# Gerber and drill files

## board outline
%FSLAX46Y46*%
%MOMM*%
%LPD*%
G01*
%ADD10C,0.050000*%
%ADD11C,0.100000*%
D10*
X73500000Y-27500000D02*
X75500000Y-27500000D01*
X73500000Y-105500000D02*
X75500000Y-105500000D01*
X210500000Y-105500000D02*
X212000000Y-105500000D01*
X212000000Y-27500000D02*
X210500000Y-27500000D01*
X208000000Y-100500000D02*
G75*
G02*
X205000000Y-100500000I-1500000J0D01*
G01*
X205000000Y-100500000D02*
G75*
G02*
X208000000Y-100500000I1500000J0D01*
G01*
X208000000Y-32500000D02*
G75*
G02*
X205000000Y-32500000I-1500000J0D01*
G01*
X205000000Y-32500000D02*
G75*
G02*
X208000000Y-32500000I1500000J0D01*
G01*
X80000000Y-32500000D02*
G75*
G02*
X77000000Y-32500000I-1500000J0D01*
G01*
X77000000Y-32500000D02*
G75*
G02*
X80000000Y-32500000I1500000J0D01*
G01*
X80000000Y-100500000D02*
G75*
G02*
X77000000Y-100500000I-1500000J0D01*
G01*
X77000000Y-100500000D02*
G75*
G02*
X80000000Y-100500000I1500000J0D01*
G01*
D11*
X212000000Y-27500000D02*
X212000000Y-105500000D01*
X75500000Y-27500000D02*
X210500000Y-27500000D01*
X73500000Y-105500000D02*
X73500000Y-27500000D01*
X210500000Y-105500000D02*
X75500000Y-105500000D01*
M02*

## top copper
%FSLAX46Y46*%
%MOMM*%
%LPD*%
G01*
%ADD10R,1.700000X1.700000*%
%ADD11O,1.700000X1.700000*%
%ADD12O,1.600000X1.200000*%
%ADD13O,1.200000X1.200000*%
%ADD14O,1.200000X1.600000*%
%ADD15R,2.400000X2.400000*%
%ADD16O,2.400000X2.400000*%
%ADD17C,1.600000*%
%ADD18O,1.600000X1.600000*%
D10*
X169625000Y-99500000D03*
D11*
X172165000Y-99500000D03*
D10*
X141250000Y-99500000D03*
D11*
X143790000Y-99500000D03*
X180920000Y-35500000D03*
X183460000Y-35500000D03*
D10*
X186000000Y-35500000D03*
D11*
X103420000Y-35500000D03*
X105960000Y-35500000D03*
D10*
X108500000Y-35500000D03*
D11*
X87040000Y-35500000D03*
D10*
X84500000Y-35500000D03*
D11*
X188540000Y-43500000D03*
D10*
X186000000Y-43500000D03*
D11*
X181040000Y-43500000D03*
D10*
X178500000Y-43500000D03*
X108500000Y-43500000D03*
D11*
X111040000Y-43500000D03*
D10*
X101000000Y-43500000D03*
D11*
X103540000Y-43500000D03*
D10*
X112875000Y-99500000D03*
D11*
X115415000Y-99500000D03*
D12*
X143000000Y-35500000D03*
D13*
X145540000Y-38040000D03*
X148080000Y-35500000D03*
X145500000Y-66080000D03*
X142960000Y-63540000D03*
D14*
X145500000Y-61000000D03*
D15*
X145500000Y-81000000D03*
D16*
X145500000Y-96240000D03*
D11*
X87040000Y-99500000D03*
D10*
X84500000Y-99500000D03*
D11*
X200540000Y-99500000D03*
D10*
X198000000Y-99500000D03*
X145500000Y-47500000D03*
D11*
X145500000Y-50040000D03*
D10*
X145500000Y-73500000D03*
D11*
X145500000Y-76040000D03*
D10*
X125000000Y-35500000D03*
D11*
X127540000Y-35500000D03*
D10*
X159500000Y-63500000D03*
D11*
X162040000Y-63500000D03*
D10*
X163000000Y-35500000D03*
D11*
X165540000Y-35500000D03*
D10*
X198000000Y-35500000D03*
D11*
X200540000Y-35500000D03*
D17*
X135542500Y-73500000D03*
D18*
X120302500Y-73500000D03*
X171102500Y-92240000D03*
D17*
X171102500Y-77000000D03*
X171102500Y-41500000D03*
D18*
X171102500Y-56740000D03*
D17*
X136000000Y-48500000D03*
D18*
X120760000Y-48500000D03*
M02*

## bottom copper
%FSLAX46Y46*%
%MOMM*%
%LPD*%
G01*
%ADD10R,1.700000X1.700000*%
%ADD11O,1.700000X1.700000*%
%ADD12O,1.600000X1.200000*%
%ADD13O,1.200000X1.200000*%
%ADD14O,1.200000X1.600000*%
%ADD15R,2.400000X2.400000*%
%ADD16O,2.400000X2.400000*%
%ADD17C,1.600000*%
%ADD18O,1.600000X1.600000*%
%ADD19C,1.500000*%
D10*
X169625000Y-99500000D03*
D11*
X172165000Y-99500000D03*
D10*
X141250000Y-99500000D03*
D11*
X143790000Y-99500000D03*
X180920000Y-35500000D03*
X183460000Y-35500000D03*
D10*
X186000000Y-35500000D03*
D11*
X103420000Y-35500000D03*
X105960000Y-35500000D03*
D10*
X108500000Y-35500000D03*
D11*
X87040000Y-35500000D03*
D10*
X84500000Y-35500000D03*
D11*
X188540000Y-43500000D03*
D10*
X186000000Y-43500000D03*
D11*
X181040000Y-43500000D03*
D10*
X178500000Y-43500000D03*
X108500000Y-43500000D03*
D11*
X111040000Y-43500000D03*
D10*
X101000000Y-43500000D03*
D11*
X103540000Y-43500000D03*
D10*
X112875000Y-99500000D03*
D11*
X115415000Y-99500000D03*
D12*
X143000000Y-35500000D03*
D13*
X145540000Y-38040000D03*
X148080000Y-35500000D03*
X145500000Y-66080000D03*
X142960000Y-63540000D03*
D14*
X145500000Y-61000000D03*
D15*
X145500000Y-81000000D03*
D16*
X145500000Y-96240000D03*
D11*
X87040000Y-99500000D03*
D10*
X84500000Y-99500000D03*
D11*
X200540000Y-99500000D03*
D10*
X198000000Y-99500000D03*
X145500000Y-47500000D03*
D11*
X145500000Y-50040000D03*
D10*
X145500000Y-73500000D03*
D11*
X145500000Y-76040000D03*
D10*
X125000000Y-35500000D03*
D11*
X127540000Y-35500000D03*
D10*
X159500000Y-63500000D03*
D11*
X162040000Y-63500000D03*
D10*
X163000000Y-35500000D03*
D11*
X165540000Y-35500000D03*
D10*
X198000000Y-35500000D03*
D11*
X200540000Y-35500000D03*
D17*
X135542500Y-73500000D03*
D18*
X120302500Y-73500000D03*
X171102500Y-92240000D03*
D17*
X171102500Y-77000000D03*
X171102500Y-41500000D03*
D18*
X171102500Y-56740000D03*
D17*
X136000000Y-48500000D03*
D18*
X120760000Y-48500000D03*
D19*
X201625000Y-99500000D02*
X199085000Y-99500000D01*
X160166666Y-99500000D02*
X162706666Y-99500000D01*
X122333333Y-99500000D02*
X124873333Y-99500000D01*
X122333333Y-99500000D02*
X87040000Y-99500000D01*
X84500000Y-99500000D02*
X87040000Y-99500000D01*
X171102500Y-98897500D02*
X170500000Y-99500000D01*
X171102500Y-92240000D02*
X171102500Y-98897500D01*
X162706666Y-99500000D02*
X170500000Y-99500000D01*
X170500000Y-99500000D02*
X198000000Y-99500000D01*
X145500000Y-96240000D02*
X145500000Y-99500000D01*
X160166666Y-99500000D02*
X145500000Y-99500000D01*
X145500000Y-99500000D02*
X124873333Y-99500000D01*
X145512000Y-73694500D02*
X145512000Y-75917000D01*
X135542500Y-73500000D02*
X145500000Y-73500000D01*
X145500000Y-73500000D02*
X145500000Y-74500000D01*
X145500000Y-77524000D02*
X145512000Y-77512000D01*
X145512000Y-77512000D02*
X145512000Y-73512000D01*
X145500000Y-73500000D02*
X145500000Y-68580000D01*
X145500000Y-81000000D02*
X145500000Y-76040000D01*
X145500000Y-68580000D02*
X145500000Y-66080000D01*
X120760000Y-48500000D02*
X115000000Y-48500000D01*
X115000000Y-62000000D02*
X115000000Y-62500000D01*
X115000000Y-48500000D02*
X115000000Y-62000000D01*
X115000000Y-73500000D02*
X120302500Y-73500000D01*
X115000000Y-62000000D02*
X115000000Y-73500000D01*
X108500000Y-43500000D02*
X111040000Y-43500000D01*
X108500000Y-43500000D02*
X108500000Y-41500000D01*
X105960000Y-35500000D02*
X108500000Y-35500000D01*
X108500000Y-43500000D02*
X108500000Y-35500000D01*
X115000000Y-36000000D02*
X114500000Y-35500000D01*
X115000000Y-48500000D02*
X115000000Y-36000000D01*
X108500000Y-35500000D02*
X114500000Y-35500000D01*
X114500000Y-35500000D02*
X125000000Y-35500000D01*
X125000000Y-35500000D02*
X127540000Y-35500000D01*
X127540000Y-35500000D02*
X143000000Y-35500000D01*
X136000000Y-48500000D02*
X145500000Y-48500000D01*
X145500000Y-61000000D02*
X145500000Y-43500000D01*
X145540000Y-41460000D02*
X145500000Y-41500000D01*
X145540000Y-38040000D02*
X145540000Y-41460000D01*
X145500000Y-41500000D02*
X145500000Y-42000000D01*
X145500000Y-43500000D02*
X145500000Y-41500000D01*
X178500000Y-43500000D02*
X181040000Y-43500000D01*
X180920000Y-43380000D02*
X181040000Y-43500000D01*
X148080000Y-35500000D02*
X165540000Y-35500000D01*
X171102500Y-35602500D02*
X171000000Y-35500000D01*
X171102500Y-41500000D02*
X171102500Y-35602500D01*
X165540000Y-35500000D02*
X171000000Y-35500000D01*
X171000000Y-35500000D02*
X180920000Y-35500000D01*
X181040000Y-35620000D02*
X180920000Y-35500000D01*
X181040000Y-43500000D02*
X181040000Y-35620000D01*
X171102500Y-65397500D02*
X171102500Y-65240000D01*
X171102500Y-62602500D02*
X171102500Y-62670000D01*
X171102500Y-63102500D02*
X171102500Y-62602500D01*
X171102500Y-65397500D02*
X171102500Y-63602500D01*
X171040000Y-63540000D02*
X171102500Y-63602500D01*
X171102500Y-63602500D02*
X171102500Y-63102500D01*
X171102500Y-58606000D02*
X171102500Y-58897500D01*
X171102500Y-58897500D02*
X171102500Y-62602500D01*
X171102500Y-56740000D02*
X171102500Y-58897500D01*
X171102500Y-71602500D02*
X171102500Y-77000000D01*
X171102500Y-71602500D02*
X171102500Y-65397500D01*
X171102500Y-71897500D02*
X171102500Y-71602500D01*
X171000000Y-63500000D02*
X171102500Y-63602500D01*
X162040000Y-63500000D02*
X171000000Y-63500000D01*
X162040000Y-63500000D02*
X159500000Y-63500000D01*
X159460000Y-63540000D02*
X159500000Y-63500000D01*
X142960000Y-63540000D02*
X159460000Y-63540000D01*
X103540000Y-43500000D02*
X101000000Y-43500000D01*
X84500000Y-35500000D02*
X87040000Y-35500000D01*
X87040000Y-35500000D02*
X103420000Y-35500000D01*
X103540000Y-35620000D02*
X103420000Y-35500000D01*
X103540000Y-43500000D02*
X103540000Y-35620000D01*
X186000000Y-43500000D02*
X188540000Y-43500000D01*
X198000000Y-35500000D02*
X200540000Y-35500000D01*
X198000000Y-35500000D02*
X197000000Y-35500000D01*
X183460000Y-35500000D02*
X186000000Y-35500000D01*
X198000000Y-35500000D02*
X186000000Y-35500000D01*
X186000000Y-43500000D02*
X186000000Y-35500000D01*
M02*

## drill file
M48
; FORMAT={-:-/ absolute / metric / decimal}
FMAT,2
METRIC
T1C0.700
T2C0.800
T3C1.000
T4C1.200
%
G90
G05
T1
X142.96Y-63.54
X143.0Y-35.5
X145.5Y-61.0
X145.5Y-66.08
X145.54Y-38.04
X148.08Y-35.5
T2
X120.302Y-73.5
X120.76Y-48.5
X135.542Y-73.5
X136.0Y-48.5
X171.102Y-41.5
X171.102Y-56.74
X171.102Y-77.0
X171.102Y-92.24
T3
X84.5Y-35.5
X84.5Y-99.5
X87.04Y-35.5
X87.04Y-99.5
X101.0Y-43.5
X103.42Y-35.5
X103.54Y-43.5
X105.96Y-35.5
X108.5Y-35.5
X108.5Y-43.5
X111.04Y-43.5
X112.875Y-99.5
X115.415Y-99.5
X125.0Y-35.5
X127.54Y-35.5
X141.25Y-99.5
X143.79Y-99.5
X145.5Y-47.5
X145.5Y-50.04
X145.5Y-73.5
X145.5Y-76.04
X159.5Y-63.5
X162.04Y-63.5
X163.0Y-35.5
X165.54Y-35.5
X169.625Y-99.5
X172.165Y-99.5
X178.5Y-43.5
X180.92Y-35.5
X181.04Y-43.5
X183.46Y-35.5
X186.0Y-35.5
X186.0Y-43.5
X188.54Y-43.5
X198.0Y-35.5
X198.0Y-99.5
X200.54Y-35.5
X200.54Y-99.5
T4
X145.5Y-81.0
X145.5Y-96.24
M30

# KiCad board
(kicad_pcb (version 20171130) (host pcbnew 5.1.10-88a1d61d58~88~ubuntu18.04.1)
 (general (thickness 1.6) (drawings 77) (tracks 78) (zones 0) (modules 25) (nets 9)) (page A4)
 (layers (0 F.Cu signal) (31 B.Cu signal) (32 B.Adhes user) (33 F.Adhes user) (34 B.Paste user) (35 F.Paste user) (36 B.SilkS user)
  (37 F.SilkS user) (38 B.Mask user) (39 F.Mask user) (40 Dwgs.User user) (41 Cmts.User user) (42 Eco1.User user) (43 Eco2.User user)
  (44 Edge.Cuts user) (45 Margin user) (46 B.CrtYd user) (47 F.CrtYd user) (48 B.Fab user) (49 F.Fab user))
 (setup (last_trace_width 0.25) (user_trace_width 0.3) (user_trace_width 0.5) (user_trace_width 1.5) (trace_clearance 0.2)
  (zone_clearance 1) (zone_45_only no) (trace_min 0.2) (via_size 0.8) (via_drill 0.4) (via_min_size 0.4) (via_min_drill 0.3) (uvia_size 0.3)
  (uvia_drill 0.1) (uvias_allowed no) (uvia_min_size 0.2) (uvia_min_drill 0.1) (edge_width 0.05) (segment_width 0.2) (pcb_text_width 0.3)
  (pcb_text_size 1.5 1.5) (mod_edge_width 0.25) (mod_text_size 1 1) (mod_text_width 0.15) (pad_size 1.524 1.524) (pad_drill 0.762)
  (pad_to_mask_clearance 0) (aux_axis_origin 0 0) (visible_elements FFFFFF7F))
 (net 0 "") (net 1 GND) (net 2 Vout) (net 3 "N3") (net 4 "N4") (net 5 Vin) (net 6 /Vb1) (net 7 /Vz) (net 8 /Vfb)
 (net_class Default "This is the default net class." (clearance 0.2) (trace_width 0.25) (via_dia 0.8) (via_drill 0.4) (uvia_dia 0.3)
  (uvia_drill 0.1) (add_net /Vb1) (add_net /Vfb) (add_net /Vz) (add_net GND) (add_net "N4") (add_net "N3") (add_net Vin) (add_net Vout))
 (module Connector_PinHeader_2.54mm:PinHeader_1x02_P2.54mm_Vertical (layer F.Cu) (at 169.625 99.5 90)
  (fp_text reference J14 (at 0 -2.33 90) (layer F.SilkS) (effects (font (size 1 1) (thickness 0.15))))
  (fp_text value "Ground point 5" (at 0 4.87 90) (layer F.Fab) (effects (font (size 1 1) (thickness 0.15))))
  (pad 1 thru_hole rect (at 0 0 90) (size 1.7 1.7) (drill 1) (layers *.Cu *.Mask) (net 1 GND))
  (pad 2 thru_hole oval (at 0 2.54 90) (size 1.7 1.7) (drill 1) (layers *.Cu *.Mask) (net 1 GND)))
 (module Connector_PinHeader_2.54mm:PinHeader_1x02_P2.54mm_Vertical (layer F.Cu) (at 141.25 99.5 90)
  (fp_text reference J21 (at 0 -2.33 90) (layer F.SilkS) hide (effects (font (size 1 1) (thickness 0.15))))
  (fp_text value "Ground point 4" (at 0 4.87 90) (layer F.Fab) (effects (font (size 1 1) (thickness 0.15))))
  (pad 1 thru_hole rect (at 0 0 90) (size 1.7 1.7) (drill 1) (layers *.Cu *.Mask) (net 1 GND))
  (pad 2 thru_hole oval (at 0 2.54 90) (size 1.7 1.7) (drill 1) (layers *.Cu *.Mask) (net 1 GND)))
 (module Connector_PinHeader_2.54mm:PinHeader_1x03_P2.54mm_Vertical (layer F.Cu) (at 186 35.5 270)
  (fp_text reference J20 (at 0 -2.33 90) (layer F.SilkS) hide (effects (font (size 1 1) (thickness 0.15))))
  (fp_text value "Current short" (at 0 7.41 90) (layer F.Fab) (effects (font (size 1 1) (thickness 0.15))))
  (pad 3 thru_hole oval (at 0 5.08 270) (size 1.7 1.7) (drill 1) (layers *.Cu *.Mask) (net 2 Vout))
  (pad 2 thru_hole oval (at 0 2.54 270) (size 1.7 1.7) (drill 1) (layers *.Cu *.Mask) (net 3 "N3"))
  (pad 1 thru_hole rect (at 0 0 270) (size 1.7 1.7) (drill 1) (layers *.Cu *.Mask) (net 3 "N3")))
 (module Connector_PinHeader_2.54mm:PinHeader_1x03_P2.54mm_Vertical (layer F.Cu) (at 108.5 35.5 270)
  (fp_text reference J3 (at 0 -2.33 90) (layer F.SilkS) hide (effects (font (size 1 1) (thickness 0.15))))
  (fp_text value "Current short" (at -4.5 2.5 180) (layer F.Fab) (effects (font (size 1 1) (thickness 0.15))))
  (pad 3 thru_hole oval (at 0 5.08 270) (size 1.7 1.7) (drill 1) (layers *.Cu *.Mask) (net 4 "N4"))
  (pad 2 thru_hole oval (at 0 2.54 270) (size 1.7 1.7) (drill 1) (layers *.Cu *.Mask) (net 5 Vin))
  (pad 1 thru_hole rect (at 0 0 270) (size 1.7 1.7) (drill 1) (layers *.Cu *.Mask) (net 5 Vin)))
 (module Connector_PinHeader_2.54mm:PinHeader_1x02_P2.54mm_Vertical (layer F.Cu) (at 84.5 35.5 90)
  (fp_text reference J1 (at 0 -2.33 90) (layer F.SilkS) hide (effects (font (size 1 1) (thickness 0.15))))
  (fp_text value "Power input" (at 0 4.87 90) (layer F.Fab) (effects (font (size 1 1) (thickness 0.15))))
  (pad 2 thru_hole oval (at 0 2.54 90) (size 1.7 1.7) (drill 1) (layers *.Cu *.Mask) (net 4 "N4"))
  (pad 1 thru_hole rect (at 0 0 90) (size 1.7 1.7) (drill 1) (layers *.Cu *.Mask) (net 4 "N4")))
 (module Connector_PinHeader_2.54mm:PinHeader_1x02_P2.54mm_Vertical (layer F.Cu) (at 186 43.5 90)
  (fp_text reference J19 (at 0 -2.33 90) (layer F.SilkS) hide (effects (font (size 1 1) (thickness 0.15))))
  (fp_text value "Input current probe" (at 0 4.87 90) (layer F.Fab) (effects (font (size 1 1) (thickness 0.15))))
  (pad 2 thru_hole oval (at 0 2.54 90) (size 1.7 1.7) (drill 1) (layers *.Cu *.Mask) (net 3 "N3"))
  (pad 1 thru_hole rect (at 0 0 90) (size 1.7 1.7) (drill 1) (layers *.Cu *.Mask) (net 3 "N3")))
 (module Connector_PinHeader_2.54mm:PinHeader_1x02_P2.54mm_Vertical (layer F.Cu) (at 178.5 43.5 90)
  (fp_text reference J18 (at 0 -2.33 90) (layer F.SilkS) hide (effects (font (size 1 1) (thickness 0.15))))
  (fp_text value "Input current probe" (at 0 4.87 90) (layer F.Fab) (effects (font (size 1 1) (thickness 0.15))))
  (pad 2 thru_hole oval (at 0 2.54 90) (size 1.7 1.7) (drill 1) (layers *.Cu *.Mask) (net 2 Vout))
  (pad 1 thru_hole rect (at 0 0 90) (size 1.7 1.7) (drill 1) (layers *.Cu *.Mask) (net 2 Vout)))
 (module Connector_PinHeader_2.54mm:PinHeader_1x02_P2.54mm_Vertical (layer F.Cu) (at 108.5 43.5 90)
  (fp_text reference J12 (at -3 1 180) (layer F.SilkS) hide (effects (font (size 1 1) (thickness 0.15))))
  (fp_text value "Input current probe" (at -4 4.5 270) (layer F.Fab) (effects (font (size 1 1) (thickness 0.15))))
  (pad 1 thru_hole rect (at 0 0 90) (size 1.7 1.7) (drill 1) (layers *.Cu *.Mask) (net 5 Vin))
  (pad 2 thru_hole oval (at 0 2.54 90) (size 1.7 1.7) (drill 1) (layers *.Cu *.Mask) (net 5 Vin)))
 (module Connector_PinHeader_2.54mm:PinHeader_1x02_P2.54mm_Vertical (layer F.Cu) (at 101 43.5 90)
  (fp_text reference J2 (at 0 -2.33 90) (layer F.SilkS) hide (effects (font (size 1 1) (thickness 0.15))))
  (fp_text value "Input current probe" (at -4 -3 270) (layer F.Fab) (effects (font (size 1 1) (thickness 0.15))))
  (pad 1 thru_hole rect (at 0 0 90) (size 1.7 1.7) (drill 1) (layers *.Cu *.Mask) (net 4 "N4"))
  (pad 2 thru_hole oval (at 0 2.54 90) (size 1.7 1.7) (drill 1) (layers *.Cu *.Mask) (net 4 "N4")))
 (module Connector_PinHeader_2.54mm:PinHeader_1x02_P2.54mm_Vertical (layer F.Cu) (at 112.875 99.5 90)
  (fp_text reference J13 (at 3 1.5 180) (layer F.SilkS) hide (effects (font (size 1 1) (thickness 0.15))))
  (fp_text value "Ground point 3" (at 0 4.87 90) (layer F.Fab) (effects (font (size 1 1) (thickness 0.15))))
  (pad 1 thru_hole rect (at 0 0 90) (size 1.7 1.7) (drill 1) (layers *.Cu *.Mask) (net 1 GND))
  (pad 2 thru_hole oval (at 0 2.54 90) (size 1.7 1.7) (drill 1) (layers *.Cu *.Mask) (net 1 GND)))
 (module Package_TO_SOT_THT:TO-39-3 (layer F.Cu) (at 143 35.5)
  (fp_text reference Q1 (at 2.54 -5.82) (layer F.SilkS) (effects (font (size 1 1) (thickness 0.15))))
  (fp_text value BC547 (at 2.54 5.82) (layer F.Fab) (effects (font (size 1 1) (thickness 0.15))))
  (pad 1 thru_hole oval (at 0 0) (size 1.6 1.2) (drill 0.7) (layers *.Cu *.Mask) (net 5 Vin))
  (pad 2 thru_hole oval (at 2.54 2.54) (size 1.2 1.2) (drill 0.7) (layers *.Cu *.Mask) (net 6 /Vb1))
  (pad 3 thru_hole oval (at 5.08 0) (size 1.2 1.2) (drill 0.7) (layers *.Cu *.Mask) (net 2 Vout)))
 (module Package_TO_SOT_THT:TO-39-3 (layer F.Cu) (at 145.5 61 270)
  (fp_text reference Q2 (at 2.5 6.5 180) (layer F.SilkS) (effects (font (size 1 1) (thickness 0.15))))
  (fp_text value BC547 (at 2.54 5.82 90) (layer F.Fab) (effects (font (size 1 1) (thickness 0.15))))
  (pad 3 thru_hole oval (at 5.08 0 270) (size 1.2 1.2) (drill 0.7) (layers *.Cu *.Mask) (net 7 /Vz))
  (pad 2 thru_hole oval (at 2.54 2.54 270) (size 1.2 1.2) (drill 0.7) (layers *.Cu *.Mask) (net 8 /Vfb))
  (pad 1 thru_hole oval (at 0 0 270) (size 1.6 1.2) (drill 0.7) (layers *.Cu *.Mask) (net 6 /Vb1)))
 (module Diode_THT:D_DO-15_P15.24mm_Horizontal (layer F.Cu) (at 145.5 81 270)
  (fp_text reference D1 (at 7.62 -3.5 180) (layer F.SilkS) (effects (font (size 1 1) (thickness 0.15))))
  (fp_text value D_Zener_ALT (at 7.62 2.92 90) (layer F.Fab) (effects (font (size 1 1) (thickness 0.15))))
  (pad 1 thru_hole rect (at 0 0 270) (size 2.4 2.4) (drill 1.2) (layers *.Cu *.Mask) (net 7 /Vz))
  (pad 2 thru_hole oval (at 15.24 0 270) (size 2.4 2.4) (drill 1.2) (layers *.Cu *.Mask) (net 1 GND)))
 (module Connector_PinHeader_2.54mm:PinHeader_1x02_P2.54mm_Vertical (layer F.Cu) (at 84.5 99.5 90)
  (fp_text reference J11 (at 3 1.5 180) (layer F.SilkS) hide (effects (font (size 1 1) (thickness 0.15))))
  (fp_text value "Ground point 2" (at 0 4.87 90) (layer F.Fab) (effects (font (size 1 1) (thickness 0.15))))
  (pad 2 thru_hole oval (at 0 2.54 90) (size 1.7 1.7) (drill 1) (layers *.Cu *.Mask) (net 1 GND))
  (pad 1 thru_hole rect (at 0 0 90) (size 1.7 1.7) (drill 1) (layers *.Cu *.Mask) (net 1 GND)))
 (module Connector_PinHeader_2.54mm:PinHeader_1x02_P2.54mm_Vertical (layer F.Cu) (at 198 99.5 90)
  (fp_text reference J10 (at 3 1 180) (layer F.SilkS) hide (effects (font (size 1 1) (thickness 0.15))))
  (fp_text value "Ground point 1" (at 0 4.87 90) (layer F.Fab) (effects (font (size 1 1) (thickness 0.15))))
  (pad 2 thru_hole oval (at 0 2.54 90) (size 1.7 1.7) (drill 1) (layers *.Cu *.Mask) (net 1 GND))
  (pad 1 thru_hole rect (at 0 0 90) (size 1.7 1.7) (drill 1) (layers *.Cu *.Mask) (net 1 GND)))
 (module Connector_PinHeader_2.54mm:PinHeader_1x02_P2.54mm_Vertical (layer F.Cu) (at 145.5 47.5)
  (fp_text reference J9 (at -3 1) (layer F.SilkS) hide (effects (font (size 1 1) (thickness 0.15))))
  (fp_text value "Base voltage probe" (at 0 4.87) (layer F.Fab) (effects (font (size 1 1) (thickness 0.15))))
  (pad 1 thru_hole rect (at 0 0) (size 1.7 1.7) (drill 1) (layers *.Cu *.Mask) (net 6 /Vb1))
  (pad 2 thru_hole oval (at 0 2.54) (size 1.7 1.7) (drill 1) (layers *.Cu *.Mask) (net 6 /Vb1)))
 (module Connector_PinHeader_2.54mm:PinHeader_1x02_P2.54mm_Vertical (layer F.Cu) (at 145.5 73.5)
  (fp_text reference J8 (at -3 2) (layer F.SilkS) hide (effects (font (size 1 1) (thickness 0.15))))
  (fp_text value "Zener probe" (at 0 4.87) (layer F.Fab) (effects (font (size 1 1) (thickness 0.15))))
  (pad 1 thru_hole rect (at 0 0) (size 1.7 1.7) (drill 1) (layers *.Cu *.Mask) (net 7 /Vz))
  (pad 2 thru_hole oval (at 0 2.54) (size 1.7 1.7) (drill 1) (layers *.Cu *.Mask) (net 7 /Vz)))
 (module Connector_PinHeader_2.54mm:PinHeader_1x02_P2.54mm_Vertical (layer F.Cu) (at 125 35.5 90)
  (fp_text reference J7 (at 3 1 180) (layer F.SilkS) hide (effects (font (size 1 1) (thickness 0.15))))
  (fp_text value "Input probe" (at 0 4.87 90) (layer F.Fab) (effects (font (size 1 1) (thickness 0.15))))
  (pad 1 thru_hole rect (at 0 0 90) (size 1.7 1.7) (drill 1) (layers *.Cu *.Mask) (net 5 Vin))
  (pad 2 thru_hole oval (at 0 2.54 90) (size 1.7 1.7) (drill 1) (layers *.Cu *.Mask) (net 5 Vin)))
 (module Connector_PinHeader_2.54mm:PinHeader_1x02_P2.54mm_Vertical (layer F.Cu) (at 159.5 63.5 90)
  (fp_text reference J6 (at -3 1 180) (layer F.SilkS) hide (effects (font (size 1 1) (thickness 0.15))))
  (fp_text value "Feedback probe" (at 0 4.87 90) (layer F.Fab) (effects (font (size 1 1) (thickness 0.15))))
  (pad 1 thru_hole rect (at 0 0 90) (size 1.7 1.7) (drill 1) (layers *.Cu *.Mask) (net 8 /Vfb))
  (pad 2 thru_hole oval (at 0 2.54 90) (size 1.7 1.7) (drill 1) (layers *.Cu *.Mask) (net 8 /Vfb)))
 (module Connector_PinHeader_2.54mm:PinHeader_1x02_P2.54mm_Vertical (layer F.Cu) (at 163 35.5 90)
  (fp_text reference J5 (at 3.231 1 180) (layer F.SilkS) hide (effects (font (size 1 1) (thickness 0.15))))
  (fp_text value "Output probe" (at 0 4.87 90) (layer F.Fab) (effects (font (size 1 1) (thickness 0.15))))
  (pad 1 thru_hole rect (at 0 0 90) (size 1.7 1.7) (drill 1) (layers *.Cu *.Mask) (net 2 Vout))
  (pad 2 thru_hole oval (at 0 2.54 90) (size 1.7 1.7) (drill 1) (layers *.Cu *.Mask) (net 2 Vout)))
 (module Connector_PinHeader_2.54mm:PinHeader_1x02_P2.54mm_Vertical (layer F.Cu) (at 198 35.5 90)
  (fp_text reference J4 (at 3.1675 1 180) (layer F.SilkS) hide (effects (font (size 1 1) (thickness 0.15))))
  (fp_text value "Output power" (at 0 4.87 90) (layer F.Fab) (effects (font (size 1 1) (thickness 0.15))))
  (pad 1 thru_hole rect (at 0 0 90) (size 1.7 1.7) (drill 1) (layers *.Cu *.Mask) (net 3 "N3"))
  (pad 2 thru_hole oval (at 0 2.54 90) (size 1.7 1.7) (drill 1) (layers *.Cu *.Mask) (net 3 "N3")))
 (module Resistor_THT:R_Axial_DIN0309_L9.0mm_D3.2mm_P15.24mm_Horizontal (layer F.Cu) (at 135.5425 73.5 180)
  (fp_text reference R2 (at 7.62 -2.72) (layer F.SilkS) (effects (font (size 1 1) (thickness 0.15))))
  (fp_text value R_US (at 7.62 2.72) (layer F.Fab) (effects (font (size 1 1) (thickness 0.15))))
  (pad 1 thru_hole circle (at 0 0 180) (size 1.6 1.6) (drill 0.8) (layers *.Cu *.Mask) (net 7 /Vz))
  (pad 2 thru_hole oval (at 15.24 0 180) (size 1.6 1.6) (drill 0.8) (layers *.Cu *.Mask) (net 5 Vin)))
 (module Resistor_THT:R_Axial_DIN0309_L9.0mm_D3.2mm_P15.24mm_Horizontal (layer F.Cu) (at 171.1025 77 270)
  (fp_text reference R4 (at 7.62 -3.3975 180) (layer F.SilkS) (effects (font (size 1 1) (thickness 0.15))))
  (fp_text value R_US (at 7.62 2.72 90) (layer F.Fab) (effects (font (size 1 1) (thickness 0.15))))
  (pad 2 thru_hole oval (at 15.24 0 270) (size 1.6 1.6) (drill 0.8) (layers *.Cu *.Mask) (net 1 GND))
  (pad 1 thru_hole circle (at 0 0 270) (size 1.6 1.6) (drill 0.8) (layers *.Cu *.Mask) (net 8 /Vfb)))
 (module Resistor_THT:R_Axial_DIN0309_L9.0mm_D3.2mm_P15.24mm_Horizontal (layer F.Cu) (at 171.1025 41.5 270)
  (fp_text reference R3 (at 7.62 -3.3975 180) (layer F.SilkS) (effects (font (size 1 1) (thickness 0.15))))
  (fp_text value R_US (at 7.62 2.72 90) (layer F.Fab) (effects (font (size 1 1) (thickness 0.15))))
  (pad 1 thru_hole circle (at 0 0 270) (size 1.6 1.6) (drill 0.8) (layers *.Cu *.Mask) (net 2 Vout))
  (pad 2 thru_hole oval (at 15.24 0 270) (size 1.6 1.6) (drill 0.8) (layers *.Cu *.Mask) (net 8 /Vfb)))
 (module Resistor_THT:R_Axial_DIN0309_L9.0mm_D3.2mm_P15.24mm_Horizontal (layer F.Cu) (at 136 48.5 180)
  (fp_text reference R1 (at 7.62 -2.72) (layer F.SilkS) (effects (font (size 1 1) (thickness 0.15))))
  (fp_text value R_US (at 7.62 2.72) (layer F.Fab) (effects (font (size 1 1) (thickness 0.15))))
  (pad 1 thru_hole circle (at 0 0 180) (size 1.6 1.6) (drill 0.8) (layers *.Cu *.Mask) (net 6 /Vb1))
  (pad 2 thru_hole oval (at 15.24 0 180) (size 1.6 1.6) (drill 0.8) (layers *.Cu *.Mask) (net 5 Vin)))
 (gr_line (start 73.5 27.5) (end 75.5 27.5) (layer Edge.Cuts) (width 0.05))
 (gr_line (start 73.5 105.5) (end 75.5 105.5) (layer Edge.Cuts) (width 0.05))
 (gr_line (start 210.5 105.5) (end 212 105.5) (layer Edge.Cuts) (width 0.05))
 (gr_line (start 212 27.5) (end 210.5 27.5) (layer Edge.Cuts) (width 0.05))
 (gr_circle (center 206.5 100.5) (end 205 100.5) (layer Edge.Cuts) (width 0.05))
 (gr_circle (center 206.5 32.5) (end 206.5 31) (layer Edge.Cuts) (width 0.05))
 (gr_circle (center 78.5 32.5) (end 78.5 31) (layer Edge.Cuts) (width 0.05))
 (gr_circle (center 78.5 100.5) (end 77 100.5) (layer Edge.Cuts) (width 0.05))
 (gr_line (start 212 27.5) (end 212 105.5) (layer Edge.Cuts) (width 0.1))
 (gr_line (start 75.5 27.5) (end 210.5 27.5) (layer Edge.Cuts) (width 0.1))
 (gr_line (start 73.5 105.5) (end 73.5 27.5) (layer Edge.Cuts) (width 0.1))
 (gr_line (start 210.5 105.5) (end 75.5 105.5) (layer Edge.Cuts) (width 0.1))
 (segment (start 201.625 99.5) (end 199.085 99.5) (width 1.5) (layer B.Cu) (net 1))
 (segment (start 160.166666 99.5) (end 162.706666 99.5) (width 1.5) (layer B.Cu) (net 1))
 (segment (start 122.333333 99.5) (end 124.873333 99.5) (width 1.5) (layer B.Cu) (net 1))
 (segment (start 122.333333 99.5) (end 87.04 99.5) (width 1.5) (layer B.Cu) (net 1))
 (segment (start 84.5 99.5) (end 87.04 99.5) (width 1.5) (layer B.Cu) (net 1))
 (segment (start 171.1025 98.8975) (end 170.5 99.5) (width 1.5) (layer B.Cu) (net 1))
 (segment (start 171.1025 92.24) (end 171.1025 98.8975) (width 1.5) (layer B.Cu) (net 1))
 (segment (start 162.706666 99.5) (end 170.5 99.5) (width 1.5) (layer B.Cu) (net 1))
 (segment (start 170.5 99.5) (end 198 99.5) (width 1.5) (layer B.Cu) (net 1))
 (segment (start 145.5 96.24) (end 145.5 99.5) (width 1.5) (layer B.Cu) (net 1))
 (segment (start 160.166666 99.5) (end 145.5 99.5) (width 1.5) (layer B.Cu) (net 1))
 (segment (start 145.5 99.5) (end 124.873333 99.5) (width 1.5) (layer B.Cu) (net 1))
 (segment (start 145.512 73.6945) (end 145.512 75.917) (width 1.5) (layer B.Cu) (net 7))
 (segment (start 135.5425 73.5) (end 145.5 73.5) (width 1.5) (layer B.Cu) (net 7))
 (segment (start 145.5 73.5) (end 145.5 74.5) (width 1.5) (layer B.Cu) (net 7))
 (segment (start 145.5 77.524) (end 145.512 77.512) (width 1.5) (layer B.Cu) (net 7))
 (segment (start 145.512 77.512) (end 145.512 73.512) (width 1.5) (layer B.Cu) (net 7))
 (segment (start 145.5 73.5) (end 145.5 68.58) (width 1.5) (layer B.Cu) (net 7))
 (segment (start 145.5 81) (end 145.5 76.04) (width 1.5) (layer B.Cu) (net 7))
 (segment (start 145.5 68.58) (end 145.5 66.08) (width 1.5) (layer B.Cu) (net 7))
 (segment (start 120.76 48.5) (end 115 48.5) (width 1.5) (layer B.Cu) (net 5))
 (segment (start 115 62) (end 115 62.5) (width 1.5) (layer B.Cu) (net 5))
 (segment (start 115 48.5) (end 115 62) (width 1.5) (layer B.Cu) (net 5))
 (segment (start 115 73.5) (end 120.3025 73.5) (width 1.5) (layer B.Cu) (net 5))
 (segment (start 115 62) (end 115 73.5) (width 1.5) (layer B.Cu) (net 5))
 (segment (start 108.5 43.5) (end 111.04 43.5) (width 1.5) (layer B.Cu) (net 5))
 (segment (start 108.5 43.5) (end 108.5 41.5) (width 1.5) (layer B.Cu) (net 5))
 (segment (start 105.96 35.5) (end 108.5 35.5) (width 1.5) (layer B.Cu) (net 5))
 (segment (start 108.5 43.5) (end 108.5 35.5) (width 1.5) (layer B.Cu) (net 5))
 (segment (start 115 36) (end 114.5 35.5) (width 1.5) (layer B.Cu) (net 5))
 (segment (start 115 48.5) (end 115 36) (width 1.5) (layer B.Cu) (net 5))
 (segment (start 108.5 35.5) (end 114.5 35.5) (width 1.5) (layer B.Cu) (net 5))
 (segment (start 114.5 35.5) (end 125 35.5) (width 1.5) (layer B.Cu) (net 5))
 (segment (start 125 35.5) (end 127.54 35.5) (width 1.5) (layer B.Cu) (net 5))
 (segment (start 127.54 35.5) (end 143 35.5) (width 1.5) (layer B.Cu) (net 5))
 (segment (start 136 48.5) (end 145.5 48.5) (width 1.5) (layer B.Cu) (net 6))
 (segment (start 145.5 61) (end 145.5 43.5) (width 1.5) (layer B.Cu) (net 6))
 (segment (start 145.54 41.46) (end 145.5 41.5) (width 1.5) (layer B.Cu) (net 6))
 (segment (start 145.54 38.04) (end 145.54 41.46) (width 1.5) (layer B.Cu) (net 6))
 (segment (start 145.5 41.5) (end 145.5 42) (width 1.5) (layer B.Cu) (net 6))
 (segment (start 145.5 43.5) (end 145.5 41.5) (width 1.5) (layer B.Cu) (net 6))
 (segment (start 178.5 43.5) (end 181.04 43.5) (width 1.5) (layer B.Cu) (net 2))
 (segment (start 180.92 43.38) (end 181.04 43.5) (width 1.5) (layer B.Cu) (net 2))
 (segment (start 148.08 35.5) (end 165.54 35.5) (width 1.5) (layer B.Cu) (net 2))
 (segment (start 171.1025 35.6025) (end 171 35.5) (width 1.5) (layer B.Cu) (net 2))
 (segment (start 171.1025 41.5) (end 171.1025 35.6025) (width 1.5) (layer B.Cu) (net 2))
 (segment (start 165.54 35.5) (end 171 35.5) (width 1.5) (layer B.Cu) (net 2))
 (segment (start 171 35.5) (end 180.92 35.5) (width 1.5) (layer B.Cu) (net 2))
 (segment (start 181.04 35.62) (end 180.92 35.5) (width 1.5) (layer B.Cu) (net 2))
 (segment (start 181.04 43.5) (end 181.04 35.62) (width 1.5) (layer B.Cu) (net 2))
 (segment (start 171.1025 65.3975) (end 171.1025 65.24) (width 1.5) (layer B.Cu) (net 8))
 (segment (start 171.1025 62.6025) (end 171.1025 62.67) (width 1.5) (layer B.Cu) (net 8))
 (segment (start 171.1025 63.1025) (end 171.1025 62.6025) (width 1.5) (layer B.Cu) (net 8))
 (segment (start 171.1025 65.3975) (end 171.1025 63.6025) (width 1.5) (layer B.Cu) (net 8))
 (segment (start 171.04 63.54) (end 171.1025 63.6025) (width 1.5) (layer B.Cu) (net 8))
 (segment (start 171.1025 63.6025) (end 171.1025 63.1025) (width 1.5) (layer B.Cu) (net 8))
 (segment (start 171.1025 58.606) (end 171.1025 58.8975) (width 1.5) (layer B.Cu) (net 8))
 (segment (start 171.1025 58.8975) (end 171.1025 62.6025) (width 1.5) (layer B.Cu) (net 8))
 (segment (start 171.1025 56.74) (end 171.1025 58.8975) (width 1.5) (layer B.Cu) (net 8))
 (segment (start 171.1025 71.6025) (end 171.1025 77) (width 1.5) (layer B.Cu) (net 8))
 (segment (start 171.1025 71.6025) (end 171.1025 65.3975) (width 1.5) (layer B.Cu) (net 8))
 (segment (start 171.1025 71.8975) (end 171.1025 71.6025) (width 1.5) (layer B.Cu) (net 8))
 (segment (start 171 63.5) (end 171.1025 63.6025) (width 1.5) (layer B.Cu) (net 8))
 (segment (start 162.04 63.5) (end 171 63.5) (width 1.5) (layer B.Cu) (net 8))
 (segment (start 162.04 63.5) (end 159.5 63.5) (width 1.5) (layer B.Cu) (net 8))
 (segment (start 159.46 63.54) (end 159.5 63.5) (width 1.5) (layer B.Cu) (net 8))
 (segment (start 142.96 63.54) (end 159.46 63.54) (width 1.5) (layer B.Cu) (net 8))
 (segment (start 103.54 43.5) (end 101 43.5) (width 1.5) (layer B.Cu) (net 4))
 (segment (start 84.5 35.5) (end 87.04 35.5) (width 1.5) (layer B.Cu) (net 4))
 (segment (start 87.04 35.5) (end 103.42 35.5) (width 1.5) (layer B.Cu) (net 4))
 (segment (start 103.54 35.62) (end 103.42 35.5) (width 1.5) (layer B.Cu) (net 4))
 (segment (start 103.54 43.5) (end 103.54 35.62) (width 1.5) (layer B.Cu) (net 4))
 (segment (start 186 43.5) (end 188.54 43.5) (width 1.5) (layer B.Cu) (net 3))
 (segment (start 198 35.5) (end 200.54 35.5) (width 1.5) (layer B.Cu) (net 3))
 (segment (start 198 35.5) (end 197 35.5) (width 1.5) (layer B.Cu) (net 3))
 (segment (start 183.46 35.5) (end 186 35.5) (width 1.5) (layer B.Cu) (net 3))
 (segment (start 198 35.5) (end 186 35.5) (width 1.5) (layer B.Cu) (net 3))
 (segment (start 186 43.5) (end 186 35.5) (width 1.5) (layer B.Cu) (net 3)))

